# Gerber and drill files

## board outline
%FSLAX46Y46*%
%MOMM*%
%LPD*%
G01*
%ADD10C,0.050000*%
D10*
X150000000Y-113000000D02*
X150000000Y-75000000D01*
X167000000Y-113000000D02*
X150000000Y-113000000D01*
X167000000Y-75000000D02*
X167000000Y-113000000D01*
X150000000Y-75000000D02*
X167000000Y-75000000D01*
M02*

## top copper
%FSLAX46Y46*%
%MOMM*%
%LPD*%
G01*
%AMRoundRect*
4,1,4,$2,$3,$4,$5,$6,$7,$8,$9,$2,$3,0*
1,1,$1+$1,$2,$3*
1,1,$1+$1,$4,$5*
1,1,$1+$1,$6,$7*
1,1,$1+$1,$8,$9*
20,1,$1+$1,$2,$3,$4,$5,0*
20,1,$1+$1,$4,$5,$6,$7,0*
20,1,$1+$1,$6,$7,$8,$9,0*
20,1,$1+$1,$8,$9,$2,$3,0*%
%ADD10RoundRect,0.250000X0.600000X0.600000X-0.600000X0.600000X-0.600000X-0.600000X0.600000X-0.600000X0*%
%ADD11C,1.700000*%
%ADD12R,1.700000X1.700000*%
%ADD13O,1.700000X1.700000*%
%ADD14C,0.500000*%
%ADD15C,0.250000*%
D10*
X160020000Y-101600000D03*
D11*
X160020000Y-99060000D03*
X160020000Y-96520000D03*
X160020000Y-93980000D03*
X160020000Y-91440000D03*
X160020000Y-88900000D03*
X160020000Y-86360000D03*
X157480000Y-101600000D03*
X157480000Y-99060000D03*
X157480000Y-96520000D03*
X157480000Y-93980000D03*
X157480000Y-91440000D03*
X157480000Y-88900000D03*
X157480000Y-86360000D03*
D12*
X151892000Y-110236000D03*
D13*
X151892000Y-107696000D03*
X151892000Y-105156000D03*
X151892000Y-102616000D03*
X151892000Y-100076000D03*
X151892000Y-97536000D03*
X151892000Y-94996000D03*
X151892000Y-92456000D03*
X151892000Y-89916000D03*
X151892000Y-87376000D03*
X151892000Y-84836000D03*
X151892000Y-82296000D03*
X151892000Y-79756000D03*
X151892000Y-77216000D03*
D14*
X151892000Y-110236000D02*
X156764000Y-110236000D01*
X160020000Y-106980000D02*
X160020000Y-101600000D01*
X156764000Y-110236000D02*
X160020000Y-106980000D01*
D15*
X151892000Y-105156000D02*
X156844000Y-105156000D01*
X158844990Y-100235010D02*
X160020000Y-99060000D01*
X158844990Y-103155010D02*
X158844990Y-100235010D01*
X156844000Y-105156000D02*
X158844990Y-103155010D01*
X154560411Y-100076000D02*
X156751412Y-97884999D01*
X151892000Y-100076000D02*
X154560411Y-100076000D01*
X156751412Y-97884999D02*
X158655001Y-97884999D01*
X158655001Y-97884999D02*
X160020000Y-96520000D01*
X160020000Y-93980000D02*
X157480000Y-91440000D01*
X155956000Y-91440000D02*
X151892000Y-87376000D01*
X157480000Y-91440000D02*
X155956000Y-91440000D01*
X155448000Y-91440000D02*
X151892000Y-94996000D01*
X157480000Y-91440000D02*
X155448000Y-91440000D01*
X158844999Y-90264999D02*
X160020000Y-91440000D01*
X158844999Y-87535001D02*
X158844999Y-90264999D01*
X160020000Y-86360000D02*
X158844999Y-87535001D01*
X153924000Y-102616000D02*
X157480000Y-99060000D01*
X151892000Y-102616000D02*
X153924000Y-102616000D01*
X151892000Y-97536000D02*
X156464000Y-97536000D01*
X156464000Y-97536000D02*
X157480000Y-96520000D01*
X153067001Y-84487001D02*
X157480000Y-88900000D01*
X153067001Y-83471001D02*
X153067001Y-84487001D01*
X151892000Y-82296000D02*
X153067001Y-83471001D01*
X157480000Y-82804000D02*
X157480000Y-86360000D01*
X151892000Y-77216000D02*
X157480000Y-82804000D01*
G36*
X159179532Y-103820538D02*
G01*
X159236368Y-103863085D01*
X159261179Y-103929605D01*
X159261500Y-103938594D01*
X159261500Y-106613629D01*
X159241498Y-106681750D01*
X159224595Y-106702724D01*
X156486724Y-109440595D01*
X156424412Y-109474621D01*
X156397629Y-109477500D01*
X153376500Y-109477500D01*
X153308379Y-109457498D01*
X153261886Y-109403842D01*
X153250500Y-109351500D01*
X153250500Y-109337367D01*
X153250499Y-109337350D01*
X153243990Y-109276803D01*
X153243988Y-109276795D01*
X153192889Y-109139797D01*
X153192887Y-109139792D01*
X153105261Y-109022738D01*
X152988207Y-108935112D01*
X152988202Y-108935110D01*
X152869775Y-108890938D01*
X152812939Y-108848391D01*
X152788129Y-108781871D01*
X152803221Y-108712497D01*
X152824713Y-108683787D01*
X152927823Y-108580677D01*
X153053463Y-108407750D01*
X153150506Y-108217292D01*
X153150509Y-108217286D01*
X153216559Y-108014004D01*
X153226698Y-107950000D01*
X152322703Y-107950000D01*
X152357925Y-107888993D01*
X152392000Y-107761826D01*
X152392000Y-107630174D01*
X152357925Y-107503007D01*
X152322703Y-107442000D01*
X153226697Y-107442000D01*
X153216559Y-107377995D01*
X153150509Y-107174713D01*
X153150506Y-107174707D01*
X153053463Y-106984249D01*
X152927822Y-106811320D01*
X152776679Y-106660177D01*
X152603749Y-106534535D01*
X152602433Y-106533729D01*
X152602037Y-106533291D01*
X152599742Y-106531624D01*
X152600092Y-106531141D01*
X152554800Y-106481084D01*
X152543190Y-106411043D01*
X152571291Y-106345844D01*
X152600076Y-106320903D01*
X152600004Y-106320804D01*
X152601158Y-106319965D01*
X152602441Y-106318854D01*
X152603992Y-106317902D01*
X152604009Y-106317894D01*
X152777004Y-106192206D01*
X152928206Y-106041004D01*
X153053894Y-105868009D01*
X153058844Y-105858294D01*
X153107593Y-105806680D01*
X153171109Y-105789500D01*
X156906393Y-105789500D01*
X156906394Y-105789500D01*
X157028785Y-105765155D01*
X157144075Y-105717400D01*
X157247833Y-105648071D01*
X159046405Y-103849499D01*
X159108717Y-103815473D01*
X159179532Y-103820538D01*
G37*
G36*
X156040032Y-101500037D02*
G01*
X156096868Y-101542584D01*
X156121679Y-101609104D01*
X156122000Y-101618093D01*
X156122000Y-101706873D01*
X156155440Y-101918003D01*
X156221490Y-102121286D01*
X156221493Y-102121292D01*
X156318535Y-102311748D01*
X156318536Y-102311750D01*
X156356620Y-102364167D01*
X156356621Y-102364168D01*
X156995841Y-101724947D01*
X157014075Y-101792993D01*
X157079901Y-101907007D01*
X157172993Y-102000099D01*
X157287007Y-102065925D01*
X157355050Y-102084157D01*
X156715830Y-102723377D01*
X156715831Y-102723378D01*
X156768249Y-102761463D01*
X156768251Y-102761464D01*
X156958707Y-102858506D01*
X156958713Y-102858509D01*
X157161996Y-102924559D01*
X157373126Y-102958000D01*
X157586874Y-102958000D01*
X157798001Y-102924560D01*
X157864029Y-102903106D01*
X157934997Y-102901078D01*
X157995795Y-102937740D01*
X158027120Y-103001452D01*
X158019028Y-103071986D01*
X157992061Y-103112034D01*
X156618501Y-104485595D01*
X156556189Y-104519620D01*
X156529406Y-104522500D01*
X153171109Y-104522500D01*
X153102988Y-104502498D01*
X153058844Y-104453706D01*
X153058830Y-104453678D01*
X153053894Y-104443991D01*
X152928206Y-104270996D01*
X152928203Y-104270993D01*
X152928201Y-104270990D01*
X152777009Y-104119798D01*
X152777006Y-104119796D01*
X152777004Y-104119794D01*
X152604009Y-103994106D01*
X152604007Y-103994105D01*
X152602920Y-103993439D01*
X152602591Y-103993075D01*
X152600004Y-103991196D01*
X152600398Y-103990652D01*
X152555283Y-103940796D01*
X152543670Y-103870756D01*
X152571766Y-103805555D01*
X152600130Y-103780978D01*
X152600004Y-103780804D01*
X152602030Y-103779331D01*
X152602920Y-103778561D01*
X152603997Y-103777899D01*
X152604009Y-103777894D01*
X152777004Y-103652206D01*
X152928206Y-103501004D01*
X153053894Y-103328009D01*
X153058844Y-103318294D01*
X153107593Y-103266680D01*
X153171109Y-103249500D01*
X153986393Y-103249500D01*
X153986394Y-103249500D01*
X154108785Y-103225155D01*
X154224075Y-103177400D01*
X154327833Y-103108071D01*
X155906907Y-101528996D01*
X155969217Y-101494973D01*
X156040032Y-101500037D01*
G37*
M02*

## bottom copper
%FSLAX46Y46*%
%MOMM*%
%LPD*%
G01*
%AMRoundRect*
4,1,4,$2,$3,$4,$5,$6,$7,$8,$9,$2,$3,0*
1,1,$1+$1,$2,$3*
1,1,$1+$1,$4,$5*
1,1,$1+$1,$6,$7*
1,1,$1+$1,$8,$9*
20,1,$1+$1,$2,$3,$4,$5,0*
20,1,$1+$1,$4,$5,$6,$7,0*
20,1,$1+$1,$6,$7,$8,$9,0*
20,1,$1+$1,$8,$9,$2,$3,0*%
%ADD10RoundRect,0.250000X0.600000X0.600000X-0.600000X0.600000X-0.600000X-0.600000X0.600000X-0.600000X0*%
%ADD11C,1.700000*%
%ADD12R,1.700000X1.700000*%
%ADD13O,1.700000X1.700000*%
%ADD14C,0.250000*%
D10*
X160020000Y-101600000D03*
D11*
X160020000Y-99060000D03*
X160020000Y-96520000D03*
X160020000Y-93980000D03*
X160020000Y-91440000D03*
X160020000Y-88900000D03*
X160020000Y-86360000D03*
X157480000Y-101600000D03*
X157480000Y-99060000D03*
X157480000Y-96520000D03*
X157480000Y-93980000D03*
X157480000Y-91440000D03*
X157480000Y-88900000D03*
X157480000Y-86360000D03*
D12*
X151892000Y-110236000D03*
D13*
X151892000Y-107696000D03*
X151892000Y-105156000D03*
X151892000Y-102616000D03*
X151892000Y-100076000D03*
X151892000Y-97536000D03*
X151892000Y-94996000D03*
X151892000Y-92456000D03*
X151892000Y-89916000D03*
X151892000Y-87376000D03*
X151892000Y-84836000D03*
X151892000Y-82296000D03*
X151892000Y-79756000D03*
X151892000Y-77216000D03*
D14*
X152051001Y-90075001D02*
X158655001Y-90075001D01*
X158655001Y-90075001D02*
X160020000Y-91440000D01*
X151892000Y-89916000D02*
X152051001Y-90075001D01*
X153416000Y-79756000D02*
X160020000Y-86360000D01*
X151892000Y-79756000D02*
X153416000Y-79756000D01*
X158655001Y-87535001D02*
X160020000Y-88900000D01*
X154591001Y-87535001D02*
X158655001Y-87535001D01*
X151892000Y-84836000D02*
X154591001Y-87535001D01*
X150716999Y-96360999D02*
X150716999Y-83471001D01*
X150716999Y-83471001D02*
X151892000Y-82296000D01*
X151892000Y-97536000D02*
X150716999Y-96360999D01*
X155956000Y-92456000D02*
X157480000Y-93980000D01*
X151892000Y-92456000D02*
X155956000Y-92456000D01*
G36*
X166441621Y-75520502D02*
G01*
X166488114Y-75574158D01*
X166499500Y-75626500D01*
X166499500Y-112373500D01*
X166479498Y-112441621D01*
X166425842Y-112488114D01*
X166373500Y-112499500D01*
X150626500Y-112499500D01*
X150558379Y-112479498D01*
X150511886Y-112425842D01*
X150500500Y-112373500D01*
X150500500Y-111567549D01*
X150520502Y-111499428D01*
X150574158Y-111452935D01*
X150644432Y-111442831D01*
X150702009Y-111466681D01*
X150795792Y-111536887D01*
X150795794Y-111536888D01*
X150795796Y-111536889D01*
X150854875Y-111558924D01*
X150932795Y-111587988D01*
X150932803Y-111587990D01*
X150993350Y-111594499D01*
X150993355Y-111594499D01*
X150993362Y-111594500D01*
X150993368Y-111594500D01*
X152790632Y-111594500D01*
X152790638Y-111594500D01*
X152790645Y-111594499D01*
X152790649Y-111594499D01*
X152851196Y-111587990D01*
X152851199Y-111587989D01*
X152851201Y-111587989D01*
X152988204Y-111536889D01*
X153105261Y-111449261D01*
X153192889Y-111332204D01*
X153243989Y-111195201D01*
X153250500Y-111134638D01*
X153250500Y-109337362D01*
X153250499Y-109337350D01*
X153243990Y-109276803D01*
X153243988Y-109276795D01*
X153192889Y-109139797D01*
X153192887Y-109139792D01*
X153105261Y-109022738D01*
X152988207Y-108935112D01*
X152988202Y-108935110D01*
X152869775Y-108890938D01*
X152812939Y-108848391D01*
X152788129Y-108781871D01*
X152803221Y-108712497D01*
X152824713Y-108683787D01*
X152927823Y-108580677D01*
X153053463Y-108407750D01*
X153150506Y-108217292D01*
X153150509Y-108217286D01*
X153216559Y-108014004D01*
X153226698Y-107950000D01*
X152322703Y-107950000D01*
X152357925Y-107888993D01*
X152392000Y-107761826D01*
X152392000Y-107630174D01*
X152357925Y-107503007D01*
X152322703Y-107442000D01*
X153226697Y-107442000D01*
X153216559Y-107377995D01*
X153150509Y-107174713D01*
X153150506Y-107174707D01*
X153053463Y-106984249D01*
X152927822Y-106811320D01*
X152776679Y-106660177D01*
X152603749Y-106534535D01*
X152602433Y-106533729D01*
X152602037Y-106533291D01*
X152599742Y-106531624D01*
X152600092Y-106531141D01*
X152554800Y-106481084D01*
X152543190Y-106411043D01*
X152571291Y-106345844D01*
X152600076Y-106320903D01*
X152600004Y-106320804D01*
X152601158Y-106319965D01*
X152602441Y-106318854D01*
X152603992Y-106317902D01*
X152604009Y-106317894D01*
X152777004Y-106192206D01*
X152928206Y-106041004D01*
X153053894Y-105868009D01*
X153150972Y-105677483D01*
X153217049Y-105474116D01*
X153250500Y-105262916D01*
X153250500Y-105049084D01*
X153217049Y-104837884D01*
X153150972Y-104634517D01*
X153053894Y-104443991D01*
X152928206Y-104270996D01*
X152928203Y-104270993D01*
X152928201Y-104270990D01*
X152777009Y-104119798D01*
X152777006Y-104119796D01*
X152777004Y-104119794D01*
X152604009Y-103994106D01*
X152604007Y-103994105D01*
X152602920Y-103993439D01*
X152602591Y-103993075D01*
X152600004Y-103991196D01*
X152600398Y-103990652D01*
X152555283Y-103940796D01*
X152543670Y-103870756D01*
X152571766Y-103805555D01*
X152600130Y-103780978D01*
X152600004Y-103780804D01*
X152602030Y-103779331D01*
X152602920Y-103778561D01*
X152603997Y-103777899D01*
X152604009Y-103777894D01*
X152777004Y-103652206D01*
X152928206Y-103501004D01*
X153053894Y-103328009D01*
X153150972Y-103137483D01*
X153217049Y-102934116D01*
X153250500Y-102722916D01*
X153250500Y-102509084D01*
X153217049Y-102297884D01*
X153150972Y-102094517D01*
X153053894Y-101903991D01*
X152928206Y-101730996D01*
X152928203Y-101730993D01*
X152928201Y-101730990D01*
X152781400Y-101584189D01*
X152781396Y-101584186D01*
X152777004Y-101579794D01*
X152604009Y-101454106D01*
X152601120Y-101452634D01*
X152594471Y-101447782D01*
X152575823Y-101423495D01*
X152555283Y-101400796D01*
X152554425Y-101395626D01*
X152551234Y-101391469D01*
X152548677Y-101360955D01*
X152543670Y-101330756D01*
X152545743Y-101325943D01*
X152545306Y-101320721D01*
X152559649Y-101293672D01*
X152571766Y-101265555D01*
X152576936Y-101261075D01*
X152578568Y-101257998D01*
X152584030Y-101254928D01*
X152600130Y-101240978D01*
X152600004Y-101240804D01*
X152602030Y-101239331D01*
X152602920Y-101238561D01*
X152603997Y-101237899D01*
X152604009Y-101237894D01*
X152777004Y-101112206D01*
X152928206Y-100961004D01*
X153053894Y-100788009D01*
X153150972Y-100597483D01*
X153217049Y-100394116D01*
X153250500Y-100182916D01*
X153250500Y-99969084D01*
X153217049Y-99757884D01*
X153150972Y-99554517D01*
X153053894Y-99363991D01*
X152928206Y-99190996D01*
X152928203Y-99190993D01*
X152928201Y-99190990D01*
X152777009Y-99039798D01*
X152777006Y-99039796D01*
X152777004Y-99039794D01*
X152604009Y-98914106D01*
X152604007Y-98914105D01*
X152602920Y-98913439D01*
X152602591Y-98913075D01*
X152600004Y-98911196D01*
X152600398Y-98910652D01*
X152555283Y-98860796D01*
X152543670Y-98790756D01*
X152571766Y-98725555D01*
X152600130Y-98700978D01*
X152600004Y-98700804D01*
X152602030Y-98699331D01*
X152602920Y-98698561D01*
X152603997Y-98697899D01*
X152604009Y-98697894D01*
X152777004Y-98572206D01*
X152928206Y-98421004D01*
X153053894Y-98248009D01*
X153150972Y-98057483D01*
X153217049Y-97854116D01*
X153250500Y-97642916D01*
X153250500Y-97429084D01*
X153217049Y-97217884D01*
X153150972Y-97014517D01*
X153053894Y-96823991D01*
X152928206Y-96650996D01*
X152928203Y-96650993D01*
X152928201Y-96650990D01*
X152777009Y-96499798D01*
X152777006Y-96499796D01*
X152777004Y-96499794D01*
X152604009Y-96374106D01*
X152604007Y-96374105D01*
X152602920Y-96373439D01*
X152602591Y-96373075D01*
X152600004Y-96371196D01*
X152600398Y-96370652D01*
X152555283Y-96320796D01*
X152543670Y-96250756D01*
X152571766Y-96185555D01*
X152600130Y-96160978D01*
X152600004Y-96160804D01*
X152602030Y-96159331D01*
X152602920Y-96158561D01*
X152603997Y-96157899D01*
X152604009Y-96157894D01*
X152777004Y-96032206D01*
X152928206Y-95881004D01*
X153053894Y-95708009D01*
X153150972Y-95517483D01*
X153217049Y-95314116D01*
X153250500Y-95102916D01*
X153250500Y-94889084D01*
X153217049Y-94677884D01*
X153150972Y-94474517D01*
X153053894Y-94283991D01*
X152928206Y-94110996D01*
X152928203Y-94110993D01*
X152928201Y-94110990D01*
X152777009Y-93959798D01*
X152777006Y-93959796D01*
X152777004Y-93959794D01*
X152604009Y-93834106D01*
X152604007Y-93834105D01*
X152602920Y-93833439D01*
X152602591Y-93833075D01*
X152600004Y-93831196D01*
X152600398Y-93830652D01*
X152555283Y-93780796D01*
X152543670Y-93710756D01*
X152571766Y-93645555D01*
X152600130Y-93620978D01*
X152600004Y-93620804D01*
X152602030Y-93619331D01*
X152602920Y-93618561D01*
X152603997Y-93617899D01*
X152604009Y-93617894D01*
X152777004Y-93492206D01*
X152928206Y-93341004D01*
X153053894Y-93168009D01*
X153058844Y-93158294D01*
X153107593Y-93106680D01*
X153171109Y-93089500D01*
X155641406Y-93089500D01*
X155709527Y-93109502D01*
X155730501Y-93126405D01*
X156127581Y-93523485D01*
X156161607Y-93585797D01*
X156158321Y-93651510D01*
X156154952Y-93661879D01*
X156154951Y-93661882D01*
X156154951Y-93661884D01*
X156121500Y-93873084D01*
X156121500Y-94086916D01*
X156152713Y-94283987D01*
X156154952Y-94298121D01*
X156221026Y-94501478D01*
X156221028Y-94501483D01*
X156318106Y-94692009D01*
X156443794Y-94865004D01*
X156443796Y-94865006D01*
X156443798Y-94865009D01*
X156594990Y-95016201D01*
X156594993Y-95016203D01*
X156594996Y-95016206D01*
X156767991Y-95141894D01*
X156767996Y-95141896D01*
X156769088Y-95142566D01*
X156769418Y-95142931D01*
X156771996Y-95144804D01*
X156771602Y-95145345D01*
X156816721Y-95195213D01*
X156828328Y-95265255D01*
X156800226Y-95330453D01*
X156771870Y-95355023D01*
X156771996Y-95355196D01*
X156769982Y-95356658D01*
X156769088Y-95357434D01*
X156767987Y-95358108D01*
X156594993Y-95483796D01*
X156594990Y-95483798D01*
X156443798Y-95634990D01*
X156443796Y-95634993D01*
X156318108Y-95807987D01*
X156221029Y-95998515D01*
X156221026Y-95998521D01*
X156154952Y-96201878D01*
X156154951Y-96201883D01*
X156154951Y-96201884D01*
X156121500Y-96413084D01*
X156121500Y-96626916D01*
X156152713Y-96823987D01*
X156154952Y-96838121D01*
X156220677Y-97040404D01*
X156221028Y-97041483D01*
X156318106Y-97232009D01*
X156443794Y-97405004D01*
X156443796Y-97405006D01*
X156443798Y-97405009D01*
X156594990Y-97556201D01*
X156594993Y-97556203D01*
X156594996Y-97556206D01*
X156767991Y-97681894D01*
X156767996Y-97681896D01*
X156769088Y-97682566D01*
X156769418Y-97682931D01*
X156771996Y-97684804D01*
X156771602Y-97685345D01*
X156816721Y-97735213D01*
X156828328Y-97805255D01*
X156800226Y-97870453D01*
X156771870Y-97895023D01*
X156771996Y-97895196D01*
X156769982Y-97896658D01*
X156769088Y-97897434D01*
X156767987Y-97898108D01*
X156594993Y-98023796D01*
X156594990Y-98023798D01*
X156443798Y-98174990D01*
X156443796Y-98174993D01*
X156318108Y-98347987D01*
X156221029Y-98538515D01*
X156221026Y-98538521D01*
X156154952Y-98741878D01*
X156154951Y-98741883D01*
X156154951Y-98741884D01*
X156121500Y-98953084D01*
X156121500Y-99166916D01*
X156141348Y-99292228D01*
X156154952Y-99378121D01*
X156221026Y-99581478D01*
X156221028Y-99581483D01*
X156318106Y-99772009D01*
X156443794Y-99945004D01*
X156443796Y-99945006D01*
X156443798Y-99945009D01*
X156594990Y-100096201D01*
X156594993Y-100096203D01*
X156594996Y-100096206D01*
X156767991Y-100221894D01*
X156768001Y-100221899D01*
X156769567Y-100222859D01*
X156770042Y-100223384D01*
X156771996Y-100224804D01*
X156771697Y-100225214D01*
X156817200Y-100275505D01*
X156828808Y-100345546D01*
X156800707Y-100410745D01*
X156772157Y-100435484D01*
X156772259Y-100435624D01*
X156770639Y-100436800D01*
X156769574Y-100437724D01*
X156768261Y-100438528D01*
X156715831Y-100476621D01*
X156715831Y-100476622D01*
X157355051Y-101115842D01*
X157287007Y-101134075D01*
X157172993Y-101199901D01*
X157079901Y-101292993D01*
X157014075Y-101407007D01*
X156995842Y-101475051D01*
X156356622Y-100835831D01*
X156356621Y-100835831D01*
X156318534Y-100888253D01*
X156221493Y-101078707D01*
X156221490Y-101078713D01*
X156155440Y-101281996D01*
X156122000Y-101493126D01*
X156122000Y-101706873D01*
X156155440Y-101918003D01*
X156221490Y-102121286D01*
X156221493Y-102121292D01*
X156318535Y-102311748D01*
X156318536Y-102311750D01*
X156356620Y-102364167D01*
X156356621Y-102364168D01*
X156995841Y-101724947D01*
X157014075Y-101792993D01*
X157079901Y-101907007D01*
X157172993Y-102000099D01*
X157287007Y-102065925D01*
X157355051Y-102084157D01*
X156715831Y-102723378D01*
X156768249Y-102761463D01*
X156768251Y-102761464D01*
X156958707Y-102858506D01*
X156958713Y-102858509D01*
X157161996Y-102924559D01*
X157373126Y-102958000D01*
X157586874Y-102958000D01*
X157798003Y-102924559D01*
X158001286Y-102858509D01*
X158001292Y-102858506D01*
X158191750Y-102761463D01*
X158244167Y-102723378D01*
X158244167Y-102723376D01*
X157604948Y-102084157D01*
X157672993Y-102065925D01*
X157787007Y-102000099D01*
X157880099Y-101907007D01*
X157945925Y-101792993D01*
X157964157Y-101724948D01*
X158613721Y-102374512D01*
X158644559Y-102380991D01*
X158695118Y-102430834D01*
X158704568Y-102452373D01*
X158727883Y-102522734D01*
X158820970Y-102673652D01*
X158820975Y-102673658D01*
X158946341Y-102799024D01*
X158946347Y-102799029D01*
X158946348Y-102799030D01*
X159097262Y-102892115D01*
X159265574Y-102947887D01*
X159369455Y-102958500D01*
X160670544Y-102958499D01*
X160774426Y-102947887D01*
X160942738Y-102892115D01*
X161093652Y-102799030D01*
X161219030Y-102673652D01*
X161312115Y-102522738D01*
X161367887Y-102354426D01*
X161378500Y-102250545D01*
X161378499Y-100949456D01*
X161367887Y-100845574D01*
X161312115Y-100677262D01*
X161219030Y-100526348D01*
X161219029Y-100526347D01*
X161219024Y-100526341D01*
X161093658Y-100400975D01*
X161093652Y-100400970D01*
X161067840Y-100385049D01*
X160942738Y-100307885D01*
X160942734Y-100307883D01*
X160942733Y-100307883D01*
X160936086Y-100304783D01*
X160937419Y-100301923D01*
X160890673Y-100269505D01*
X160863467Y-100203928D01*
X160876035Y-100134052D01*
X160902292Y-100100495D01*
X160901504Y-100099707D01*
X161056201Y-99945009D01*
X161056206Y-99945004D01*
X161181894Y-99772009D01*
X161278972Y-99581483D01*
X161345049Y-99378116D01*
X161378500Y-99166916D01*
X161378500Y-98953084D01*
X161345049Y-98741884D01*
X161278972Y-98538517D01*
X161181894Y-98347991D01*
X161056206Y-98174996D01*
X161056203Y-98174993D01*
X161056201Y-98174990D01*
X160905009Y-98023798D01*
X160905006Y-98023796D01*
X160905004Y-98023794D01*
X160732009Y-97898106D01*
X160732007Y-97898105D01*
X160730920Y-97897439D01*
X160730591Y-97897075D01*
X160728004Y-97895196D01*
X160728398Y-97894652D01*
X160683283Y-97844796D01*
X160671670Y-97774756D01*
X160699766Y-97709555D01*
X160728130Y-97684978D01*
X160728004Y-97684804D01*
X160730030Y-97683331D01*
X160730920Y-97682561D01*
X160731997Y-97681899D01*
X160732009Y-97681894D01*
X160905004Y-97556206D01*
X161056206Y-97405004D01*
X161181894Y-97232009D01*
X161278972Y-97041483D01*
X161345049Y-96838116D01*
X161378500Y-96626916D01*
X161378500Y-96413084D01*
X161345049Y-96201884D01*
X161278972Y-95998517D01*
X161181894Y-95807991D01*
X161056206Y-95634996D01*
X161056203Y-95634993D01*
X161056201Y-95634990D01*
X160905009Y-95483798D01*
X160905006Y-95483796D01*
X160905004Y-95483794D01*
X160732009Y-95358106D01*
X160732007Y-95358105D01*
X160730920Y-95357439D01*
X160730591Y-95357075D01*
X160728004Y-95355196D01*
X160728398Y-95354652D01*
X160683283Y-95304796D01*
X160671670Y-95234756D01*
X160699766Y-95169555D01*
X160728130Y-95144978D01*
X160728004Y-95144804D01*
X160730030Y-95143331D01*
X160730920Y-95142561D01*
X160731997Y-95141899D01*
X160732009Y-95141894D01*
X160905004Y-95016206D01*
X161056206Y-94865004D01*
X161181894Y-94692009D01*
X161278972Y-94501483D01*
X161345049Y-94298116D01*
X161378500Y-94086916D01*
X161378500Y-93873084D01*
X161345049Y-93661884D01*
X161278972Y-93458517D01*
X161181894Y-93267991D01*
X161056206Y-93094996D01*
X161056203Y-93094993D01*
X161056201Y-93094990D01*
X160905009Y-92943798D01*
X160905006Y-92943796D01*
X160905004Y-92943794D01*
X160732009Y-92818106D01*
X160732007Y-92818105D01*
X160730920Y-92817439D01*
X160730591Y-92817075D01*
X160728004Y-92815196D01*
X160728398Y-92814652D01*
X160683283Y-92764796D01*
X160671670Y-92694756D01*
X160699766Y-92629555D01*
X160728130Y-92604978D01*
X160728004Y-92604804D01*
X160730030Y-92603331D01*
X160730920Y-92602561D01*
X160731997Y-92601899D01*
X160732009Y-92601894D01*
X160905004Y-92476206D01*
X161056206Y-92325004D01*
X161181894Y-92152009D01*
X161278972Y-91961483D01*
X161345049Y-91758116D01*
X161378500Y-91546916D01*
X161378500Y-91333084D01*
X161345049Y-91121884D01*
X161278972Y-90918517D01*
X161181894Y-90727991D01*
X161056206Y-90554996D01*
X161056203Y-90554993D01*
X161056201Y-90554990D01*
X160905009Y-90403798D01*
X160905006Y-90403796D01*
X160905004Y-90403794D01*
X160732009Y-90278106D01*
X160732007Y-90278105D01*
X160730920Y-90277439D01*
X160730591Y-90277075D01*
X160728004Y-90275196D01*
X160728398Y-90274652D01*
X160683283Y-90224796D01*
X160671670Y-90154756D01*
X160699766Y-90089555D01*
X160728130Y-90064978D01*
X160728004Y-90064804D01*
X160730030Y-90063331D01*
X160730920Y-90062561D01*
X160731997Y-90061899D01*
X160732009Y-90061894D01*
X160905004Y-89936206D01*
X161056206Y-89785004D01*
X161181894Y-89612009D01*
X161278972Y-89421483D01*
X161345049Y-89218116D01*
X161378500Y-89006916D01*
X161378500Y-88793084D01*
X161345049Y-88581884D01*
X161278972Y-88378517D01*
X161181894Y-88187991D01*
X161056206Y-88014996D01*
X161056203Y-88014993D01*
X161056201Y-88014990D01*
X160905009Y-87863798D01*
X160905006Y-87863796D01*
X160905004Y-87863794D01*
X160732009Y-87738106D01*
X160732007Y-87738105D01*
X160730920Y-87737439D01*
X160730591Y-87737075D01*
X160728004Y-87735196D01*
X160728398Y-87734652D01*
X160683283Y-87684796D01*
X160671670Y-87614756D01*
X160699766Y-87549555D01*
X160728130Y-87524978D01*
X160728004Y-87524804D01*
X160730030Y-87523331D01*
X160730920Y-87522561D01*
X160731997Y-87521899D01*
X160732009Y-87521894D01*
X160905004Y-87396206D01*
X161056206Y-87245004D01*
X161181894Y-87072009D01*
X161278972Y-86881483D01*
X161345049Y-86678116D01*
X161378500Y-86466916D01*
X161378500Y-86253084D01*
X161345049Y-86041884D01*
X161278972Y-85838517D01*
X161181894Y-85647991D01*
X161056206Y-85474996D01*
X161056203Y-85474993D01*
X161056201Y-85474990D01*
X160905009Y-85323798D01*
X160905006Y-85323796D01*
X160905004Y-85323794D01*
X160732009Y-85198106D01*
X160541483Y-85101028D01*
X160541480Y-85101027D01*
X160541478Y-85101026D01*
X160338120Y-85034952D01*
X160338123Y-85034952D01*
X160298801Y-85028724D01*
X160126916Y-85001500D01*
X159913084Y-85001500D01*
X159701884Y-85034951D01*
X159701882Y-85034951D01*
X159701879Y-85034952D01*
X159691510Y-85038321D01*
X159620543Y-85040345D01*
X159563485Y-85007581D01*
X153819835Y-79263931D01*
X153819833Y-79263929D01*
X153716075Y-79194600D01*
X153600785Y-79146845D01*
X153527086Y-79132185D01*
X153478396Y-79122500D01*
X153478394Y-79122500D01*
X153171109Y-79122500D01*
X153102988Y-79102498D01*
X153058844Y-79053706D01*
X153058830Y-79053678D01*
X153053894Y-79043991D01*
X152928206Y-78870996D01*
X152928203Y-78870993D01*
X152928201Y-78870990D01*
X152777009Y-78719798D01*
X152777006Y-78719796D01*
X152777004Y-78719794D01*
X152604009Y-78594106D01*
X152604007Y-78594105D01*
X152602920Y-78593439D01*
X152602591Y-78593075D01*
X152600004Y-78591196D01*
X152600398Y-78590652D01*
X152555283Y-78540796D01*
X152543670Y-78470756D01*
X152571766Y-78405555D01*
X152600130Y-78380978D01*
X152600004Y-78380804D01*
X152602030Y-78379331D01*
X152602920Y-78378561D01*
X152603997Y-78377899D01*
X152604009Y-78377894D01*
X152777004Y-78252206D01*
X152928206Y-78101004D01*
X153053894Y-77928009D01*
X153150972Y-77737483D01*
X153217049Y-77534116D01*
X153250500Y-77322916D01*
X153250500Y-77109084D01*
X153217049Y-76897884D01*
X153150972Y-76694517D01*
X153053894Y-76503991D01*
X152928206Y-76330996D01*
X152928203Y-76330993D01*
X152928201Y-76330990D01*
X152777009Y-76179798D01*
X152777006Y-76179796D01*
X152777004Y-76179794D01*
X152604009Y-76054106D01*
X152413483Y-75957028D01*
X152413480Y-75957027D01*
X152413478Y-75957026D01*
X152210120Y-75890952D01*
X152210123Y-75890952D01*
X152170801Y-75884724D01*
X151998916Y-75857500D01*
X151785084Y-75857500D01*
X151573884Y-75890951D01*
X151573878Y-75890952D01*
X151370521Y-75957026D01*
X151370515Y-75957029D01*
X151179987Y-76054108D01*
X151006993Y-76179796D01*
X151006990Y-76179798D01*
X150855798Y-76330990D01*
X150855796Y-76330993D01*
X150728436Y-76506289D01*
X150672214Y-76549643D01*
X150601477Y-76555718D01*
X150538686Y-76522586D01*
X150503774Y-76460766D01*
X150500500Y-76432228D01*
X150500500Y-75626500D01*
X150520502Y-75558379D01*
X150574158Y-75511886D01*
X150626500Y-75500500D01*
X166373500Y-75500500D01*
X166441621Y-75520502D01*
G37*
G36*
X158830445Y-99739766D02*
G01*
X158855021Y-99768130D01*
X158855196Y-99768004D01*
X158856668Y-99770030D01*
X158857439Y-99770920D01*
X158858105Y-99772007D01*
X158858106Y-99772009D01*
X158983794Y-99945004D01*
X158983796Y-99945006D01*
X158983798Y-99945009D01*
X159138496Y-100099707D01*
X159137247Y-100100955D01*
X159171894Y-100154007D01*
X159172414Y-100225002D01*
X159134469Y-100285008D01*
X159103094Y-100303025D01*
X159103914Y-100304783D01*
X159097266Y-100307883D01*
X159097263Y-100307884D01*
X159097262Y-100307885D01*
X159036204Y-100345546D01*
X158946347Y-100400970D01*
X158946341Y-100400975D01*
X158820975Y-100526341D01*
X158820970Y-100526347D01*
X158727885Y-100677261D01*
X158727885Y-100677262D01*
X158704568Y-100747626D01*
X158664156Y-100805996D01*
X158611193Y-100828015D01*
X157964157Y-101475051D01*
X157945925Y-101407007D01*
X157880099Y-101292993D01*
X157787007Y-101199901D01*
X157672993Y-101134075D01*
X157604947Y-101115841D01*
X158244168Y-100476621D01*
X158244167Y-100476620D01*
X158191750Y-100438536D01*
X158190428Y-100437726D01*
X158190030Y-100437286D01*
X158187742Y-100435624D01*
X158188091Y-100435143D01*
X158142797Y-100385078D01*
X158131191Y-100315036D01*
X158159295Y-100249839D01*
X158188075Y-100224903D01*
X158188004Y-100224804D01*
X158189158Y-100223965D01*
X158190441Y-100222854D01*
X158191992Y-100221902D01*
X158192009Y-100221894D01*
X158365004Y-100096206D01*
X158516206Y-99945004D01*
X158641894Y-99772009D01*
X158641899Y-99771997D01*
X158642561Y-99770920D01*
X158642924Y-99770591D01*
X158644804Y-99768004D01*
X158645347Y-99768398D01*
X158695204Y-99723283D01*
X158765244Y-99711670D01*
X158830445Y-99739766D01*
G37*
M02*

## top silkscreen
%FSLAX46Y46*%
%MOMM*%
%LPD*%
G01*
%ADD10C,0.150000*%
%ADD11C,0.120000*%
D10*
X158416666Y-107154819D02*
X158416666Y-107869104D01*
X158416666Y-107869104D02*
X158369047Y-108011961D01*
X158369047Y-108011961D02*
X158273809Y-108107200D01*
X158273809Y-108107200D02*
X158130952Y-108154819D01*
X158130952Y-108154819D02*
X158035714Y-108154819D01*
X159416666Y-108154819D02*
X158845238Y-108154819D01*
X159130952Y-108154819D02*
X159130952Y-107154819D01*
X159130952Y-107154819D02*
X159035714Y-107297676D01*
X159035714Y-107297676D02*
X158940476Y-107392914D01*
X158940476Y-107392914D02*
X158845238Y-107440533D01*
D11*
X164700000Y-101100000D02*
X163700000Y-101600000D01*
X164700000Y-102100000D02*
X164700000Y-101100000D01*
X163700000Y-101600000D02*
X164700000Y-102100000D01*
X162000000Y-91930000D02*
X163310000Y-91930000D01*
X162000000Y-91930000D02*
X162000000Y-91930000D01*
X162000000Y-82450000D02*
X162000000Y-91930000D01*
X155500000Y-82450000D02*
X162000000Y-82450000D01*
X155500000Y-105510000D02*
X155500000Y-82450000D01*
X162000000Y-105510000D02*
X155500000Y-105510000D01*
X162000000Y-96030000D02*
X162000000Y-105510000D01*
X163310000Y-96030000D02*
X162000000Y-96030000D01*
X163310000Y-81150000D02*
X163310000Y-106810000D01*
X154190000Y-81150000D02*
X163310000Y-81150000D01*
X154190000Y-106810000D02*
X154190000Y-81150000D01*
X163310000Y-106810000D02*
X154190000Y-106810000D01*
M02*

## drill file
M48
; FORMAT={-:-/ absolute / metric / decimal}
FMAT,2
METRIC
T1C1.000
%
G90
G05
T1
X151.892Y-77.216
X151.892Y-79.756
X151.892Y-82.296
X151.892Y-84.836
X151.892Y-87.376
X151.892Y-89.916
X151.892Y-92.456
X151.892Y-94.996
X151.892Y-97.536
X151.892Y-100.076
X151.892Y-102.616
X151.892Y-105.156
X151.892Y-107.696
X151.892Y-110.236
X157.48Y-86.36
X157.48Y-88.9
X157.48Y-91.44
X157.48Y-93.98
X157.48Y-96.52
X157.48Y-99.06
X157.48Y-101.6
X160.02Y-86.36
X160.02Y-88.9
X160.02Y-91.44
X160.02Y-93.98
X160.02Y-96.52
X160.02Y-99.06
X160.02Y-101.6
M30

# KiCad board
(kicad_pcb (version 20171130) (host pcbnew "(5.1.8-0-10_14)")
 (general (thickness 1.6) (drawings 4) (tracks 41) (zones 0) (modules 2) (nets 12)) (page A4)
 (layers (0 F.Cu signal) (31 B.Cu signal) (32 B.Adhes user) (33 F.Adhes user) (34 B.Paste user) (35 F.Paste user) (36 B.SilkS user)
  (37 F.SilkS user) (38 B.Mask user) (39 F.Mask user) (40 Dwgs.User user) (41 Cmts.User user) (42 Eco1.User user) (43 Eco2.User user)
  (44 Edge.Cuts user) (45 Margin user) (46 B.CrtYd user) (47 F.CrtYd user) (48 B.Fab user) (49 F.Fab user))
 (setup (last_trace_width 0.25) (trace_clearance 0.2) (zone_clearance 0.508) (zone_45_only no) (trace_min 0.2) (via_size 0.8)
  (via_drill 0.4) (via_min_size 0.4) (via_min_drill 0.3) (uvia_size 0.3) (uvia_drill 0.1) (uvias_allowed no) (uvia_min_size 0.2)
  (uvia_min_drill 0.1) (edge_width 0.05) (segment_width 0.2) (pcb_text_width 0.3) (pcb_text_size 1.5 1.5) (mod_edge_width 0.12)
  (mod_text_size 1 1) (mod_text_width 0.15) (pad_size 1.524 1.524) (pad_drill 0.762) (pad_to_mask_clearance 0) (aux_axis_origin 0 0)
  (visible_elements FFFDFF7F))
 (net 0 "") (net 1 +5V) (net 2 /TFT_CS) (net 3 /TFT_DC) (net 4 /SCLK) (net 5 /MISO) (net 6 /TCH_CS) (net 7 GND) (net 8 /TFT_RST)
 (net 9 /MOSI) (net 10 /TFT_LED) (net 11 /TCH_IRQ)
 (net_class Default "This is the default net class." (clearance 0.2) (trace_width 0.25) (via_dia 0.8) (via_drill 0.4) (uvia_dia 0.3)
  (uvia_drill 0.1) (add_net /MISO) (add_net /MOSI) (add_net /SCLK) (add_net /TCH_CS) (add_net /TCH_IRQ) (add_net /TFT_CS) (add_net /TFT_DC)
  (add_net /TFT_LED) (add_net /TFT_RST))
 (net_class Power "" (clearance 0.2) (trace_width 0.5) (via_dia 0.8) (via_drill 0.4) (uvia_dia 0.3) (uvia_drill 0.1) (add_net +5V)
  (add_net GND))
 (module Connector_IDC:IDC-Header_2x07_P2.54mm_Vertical (layer F.Cu) (at 160.02 101.6 180)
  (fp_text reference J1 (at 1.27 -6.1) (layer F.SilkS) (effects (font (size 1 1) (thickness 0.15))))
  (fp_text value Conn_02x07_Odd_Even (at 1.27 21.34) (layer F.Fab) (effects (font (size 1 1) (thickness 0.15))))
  (fp_line (start -4.68 0.5) (end -3.68 0) (layer F.SilkS) (width 0.12))
  (fp_line (start -4.68 -0.5) (end -4.68 0.5) (layer F.SilkS) (width 0.12))
  (fp_line (start -3.68 0) (end -4.68 -0.5) (layer F.SilkS) (width 0.12))
  (fp_line (start -1.98 9.67) (end -3.29 9.67) (layer F.SilkS) (width 0.12))
  (fp_line (start -1.98 9.67) (end -1.98 9.67) (layer F.SilkS) (width 0.12))
  (fp_line (start -1.98 19.15) (end -1.98 9.67) (layer F.SilkS) (width 0.12))
  (fp_line (start 4.52 19.15) (end -1.98 19.15) (layer F.SilkS) (width 0.12))
  (fp_line (start 4.52 -3.91) (end 4.52 19.15) (layer F.SilkS) (width 0.12))
  (fp_line (start -1.98 -3.91) (end 4.52 -3.91) (layer F.SilkS) (width 0.12))
  (fp_line (start -1.98 5.57) (end -1.98 -3.91) (layer F.SilkS) (width 0.12))
  (fp_line (start -3.29 5.57) (end -1.98 5.57) (layer F.SilkS) (width 0.12))
  (fp_line (start -3.29 20.45) (end -3.29 -5.21) (layer F.SilkS) (width 0.12))
  (fp_line (start 5.83 20.45) (end -3.29 20.45) (layer F.SilkS) (width 0.12))
  (fp_line (start 5.83 -5.21) (end 5.83 20.45) (layer F.SilkS) (width 0.12))
  (fp_line (start -3.29 -5.21) (end 5.83 -5.21) (layer F.SilkS) (width 0.12))
  (pad 1 thru_hole roundrect (at 0 0 180) (size 1.7 1.7) (drill 1) (layers *.Cu *.Mask) (roundrect_rratio 0.147059) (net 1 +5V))
  (pad 3 thru_hole circle (at 0 2.54 180) (size 1.7 1.7) (drill 1) (layers *.Cu *.Mask) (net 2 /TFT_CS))
  (pad 5 thru_hole circle (at 0 5.08 180) (size 1.7 1.7) (drill 1) (layers *.Cu *.Mask) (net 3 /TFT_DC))
  (pad 7 thru_hole circle (at 0 7.62 180) (size 1.7 1.7) (drill 1) (layers *.Cu *.Mask) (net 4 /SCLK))
  (pad 9 thru_hole circle (at 0 10.16 180) (size 1.7 1.7) (drill 1) (layers *.Cu *.Mask) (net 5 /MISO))
  (pad 11 thru_hole circle (at 0 12.7 180) (size 1.7 1.7) (drill 1) (layers *.Cu *.Mask) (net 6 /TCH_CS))
  (pad 13 thru_hole circle (at 0 15.24 180) (size 1.7 1.7) (drill 1) (layers *.Cu *.Mask) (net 5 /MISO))
  (pad 2 thru_hole circle (at 2.54 0 180) (size 1.7 1.7) (drill 1) (layers *.Cu *.Mask) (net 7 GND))
  (pad 4 thru_hole circle (at 2.54 2.54 180) (size 1.7 1.7) (drill 1) (layers *.Cu *.Mask) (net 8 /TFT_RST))
  (pad 6 thru_hole circle (at 2.54 5.08 180) (size 1.7 1.7) (drill 1) (layers *.Cu *.Mask) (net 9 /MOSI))
  (pad 8 thru_hole circle (at 2.54 7.62 180) (size 1.7 1.7) (drill 1) (layers *.Cu *.Mask) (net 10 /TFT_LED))
  (pad 10 thru_hole circle (at 2.54 10.16 180) (size 1.7 1.7) (drill 1) (layers *.Cu *.Mask) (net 4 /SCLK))
  (pad 12 thru_hole circle (at 2.54 12.7 180) (size 1.7 1.7) (drill 1) (layers *.Cu *.Mask) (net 9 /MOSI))
  (pad 14 thru_hole circle (at 2.54 15.24 180) (size 1.7 1.7) (drill 1) (layers *.Cu *.Mask) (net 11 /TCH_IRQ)))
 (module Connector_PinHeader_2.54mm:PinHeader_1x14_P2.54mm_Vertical (layer B.Cu) (at 151.892 110.236)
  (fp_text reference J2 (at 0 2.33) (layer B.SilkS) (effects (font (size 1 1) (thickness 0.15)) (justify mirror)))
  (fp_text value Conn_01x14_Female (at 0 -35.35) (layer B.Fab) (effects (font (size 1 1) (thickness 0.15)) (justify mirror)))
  (pad 1 thru_hole rect (at 0 0) (size 1.7 1.7) (drill 1) (layers *.Cu *.Mask) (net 1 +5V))
  (pad 2 thru_hole oval (at 0 -2.54) (size 1.7 1.7) (drill 1) (layers *.Cu *.Mask) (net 7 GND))
  (pad 3 thru_hole oval (at 0 -5.08) (size 1.7 1.7) (drill 1) (layers *.Cu *.Mask) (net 2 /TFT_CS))
  (pad 4 thru_hole oval (at 0 -7.62) (size 1.7 1.7) (drill 1) (layers *.Cu *.Mask) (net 8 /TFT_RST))
  (pad 5 thru_hole oval (at 0 -10.16) (size 1.7 1.7) (drill 1) (layers *.Cu *.Mask) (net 3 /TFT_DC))
  (pad 6 thru_hole oval (at 0 -12.7) (size 1.7 1.7) (drill 1) (layers *.Cu *.Mask) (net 9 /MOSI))
  (pad 7 thru_hole oval (at 0 -15.24) (size 1.7 1.7) (drill 1) (layers *.Cu *.Mask) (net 4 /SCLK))
  (pad 8 thru_hole oval (at 0 -17.78) (size 1.7 1.7) (drill 1) (layers *.Cu *.Mask) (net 10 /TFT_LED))
  (pad 9 thru_hole oval (at 0 -20.32) (size 1.7 1.7) (drill 1) (layers *.Cu *.Mask) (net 5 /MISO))
  (pad 10 thru_hole oval (at 0 -22.86) (size 1.7 1.7) (drill 1) (layers *.Cu *.Mask) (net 4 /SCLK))
  (pad 11 thru_hole oval (at 0 -25.4) (size 1.7 1.7) (drill 1) (layers *.Cu *.Mask) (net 6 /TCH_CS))
  (pad 12 thru_hole oval (at 0 -27.94) (size 1.7 1.7) (drill 1) (layers *.Cu *.Mask) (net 9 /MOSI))
  (pad 13 thru_hole oval (at 0 -30.48) (size 1.7 1.7) (drill 1) (layers *.Cu *.Mask) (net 5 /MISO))
  (pad 14 thru_hole oval (at 0 -33.02) (size 1.7 1.7) (drill 1) (layers *.Cu *.Mask) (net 11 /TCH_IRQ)))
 (gr_line (start 150 113) (end 150 75) (layer Edge.Cuts) (width 0.05))
 (gr_line (start 167 113) (end 150 113) (layer Edge.Cuts) (width 0.05))
 (gr_line (start 167 75) (end 167 113) (layer Edge.Cuts) (width 0.05))
 (gr_line (start 150 75) (end 167 75) (layer Edge.Cuts) (width 0.05))
 (segment (start 151.892 110.236) (end 156.764 110.236) (width 0.5) (layer F.Cu) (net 1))
 (segment (start 160.02 106.98) (end 160.02 101.6) (width 0.5) (layer F.Cu) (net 1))
 (segment (start 156.764 110.236) (end 160.02 106.98) (width 0.5) (layer F.Cu) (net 1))
 (segment (start 151.892 105.156) (end 156.844 105.156) (width 0.25) (layer F.Cu) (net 2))
 (segment (start 158.84499 100.23501) (end 160.02 99.06) (width 0.25) (layer F.Cu) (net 2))
 (segment (start 158.84499 103.15501) (end 158.84499 100.23501) (width 0.25) (layer F.Cu) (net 2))
 (segment (start 156.844 105.156) (end 158.84499 103.15501) (width 0.25) (layer F.Cu) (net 2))
 (segment (start 154.560411 100.076) (end 156.751412 97.884999) (width 0.25) (layer F.Cu) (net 3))
 (segment (start 151.892 100.076) (end 154.560411 100.076) (width 0.25) (layer F.Cu) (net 3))
 (segment (start 156.751412 97.884999) (end 158.655001 97.884999) (width 0.25) (layer F.Cu) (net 3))
 (segment (start 158.655001 97.884999) (end 160.02 96.52) (width 0.25) (layer F.Cu) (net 3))
 (segment (start 160.02 93.98) (end 157.48 91.44) (width 0.25) (layer F.Cu) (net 4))
 (segment (start 155.956 91.44) (end 151.892 87.376) (width 0.25) (layer F.Cu) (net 4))
 (segment (start 157.48 91.44) (end 155.956 91.44) (width 0.25) (layer F.Cu) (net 4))
 (segment (start 155.448 91.44) (end 151.892 94.996) (width 0.25) (layer F.Cu) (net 4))
 (segment (start 157.48 91.44) (end 155.448 91.44) (width 0.25) (layer F.Cu) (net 4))
 (segment (start 158.844999 90.264999) (end 160.02 91.44) (width 0.25) (layer F.Cu) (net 5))
 (segment (start 158.844999 87.535001) (end 158.844999 90.264999) (width 0.25) (layer F.Cu) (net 5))
 (segment (start 160.02 86.36) (end 158.844999 87.535001) (width 0.25) (layer F.Cu) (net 5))
 (segment (start 152.051001 90.075001) (end 158.655001 90.075001) (width 0.25) (layer B.Cu) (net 5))
 (segment (start 158.655001 90.075001) (end 160.02 91.44) (width 0.25) (layer B.Cu) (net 5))
 (segment (start 151.892 89.916) (end 152.051001 90.075001) (width 0.25) (layer B.Cu) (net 5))
 (segment (start 153.416 79.756) (end 160.02 86.36) (width 0.25) (layer B.Cu) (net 5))
 (segment (start 151.892 79.756) (end 153.416 79.756) (width 0.25) (layer B.Cu) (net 5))
 (segment (start 158.655001 87.535001) (end 160.02 88.9) (width 0.25) (layer B.Cu) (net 6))
 (segment (start 154.591001 87.535001) (end 158.655001 87.535001) (width 0.25) (layer B.Cu) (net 6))
 (segment (start 151.892 84.836) (end 154.591001 87.535001) (width 0.25) (layer B.Cu) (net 6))
 (segment (start 153.924 102.616) (end 157.48 99.06) (width 0.25) (layer F.Cu) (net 8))
 (segment (start 151.892 102.616) (end 153.924 102.616) (width 0.25) (layer F.Cu) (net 8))
 (segment (start 151.892 97.536) (end 156.464 97.536) (width 0.25) (layer F.Cu) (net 9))
 (segment (start 156.464 97.536) (end 157.48 96.52) (width 0.25) (layer F.Cu) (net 9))
 (segment (start 153.067001 84.487001) (end 157.48 88.9) (width 0.25) (layer F.Cu) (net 9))
 (segment (start 153.067001 83.471001) (end 153.067001 84.487001) (width 0.25) (layer F.Cu) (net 9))
 (segment (start 151.892 82.296) (end 153.067001 83.471001) (width 0.25) (layer F.Cu) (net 9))
 (segment (start 150.716999 96.360999) (end 150.716999 83.471001) (width 0.25) (layer B.Cu) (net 9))
 (segment (start 150.716999 83.471001) (end 151.892 82.296) (width 0.25) (layer B.Cu) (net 9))
 (segment (start 151.892 97.536) (end 150.716999 96.360999) (width 0.25) (layer B.Cu) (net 9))
 (segment (start 155.956 92.456) (end 157.48 93.98) (width 0.25) (layer B.Cu) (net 10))
 (segment (start 151.892 92.456) (end 155.956 92.456) (width 0.25) (layer B.Cu) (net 10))
 (segment (start 157.48 82.804) (end 157.48 86.36) (width 0.25) (layer F.Cu) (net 11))
 (segment (start 151.892 77.216) (end 157.48 82.804) (width 0.25) (layer F.Cu) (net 11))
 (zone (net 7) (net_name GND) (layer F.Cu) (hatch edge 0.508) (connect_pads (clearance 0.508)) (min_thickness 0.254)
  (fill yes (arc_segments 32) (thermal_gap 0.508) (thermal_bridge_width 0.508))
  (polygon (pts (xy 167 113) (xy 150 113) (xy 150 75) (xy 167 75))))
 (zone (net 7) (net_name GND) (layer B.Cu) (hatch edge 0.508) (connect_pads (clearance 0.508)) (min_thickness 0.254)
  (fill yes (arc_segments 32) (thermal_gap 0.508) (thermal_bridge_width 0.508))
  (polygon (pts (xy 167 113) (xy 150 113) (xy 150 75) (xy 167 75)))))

